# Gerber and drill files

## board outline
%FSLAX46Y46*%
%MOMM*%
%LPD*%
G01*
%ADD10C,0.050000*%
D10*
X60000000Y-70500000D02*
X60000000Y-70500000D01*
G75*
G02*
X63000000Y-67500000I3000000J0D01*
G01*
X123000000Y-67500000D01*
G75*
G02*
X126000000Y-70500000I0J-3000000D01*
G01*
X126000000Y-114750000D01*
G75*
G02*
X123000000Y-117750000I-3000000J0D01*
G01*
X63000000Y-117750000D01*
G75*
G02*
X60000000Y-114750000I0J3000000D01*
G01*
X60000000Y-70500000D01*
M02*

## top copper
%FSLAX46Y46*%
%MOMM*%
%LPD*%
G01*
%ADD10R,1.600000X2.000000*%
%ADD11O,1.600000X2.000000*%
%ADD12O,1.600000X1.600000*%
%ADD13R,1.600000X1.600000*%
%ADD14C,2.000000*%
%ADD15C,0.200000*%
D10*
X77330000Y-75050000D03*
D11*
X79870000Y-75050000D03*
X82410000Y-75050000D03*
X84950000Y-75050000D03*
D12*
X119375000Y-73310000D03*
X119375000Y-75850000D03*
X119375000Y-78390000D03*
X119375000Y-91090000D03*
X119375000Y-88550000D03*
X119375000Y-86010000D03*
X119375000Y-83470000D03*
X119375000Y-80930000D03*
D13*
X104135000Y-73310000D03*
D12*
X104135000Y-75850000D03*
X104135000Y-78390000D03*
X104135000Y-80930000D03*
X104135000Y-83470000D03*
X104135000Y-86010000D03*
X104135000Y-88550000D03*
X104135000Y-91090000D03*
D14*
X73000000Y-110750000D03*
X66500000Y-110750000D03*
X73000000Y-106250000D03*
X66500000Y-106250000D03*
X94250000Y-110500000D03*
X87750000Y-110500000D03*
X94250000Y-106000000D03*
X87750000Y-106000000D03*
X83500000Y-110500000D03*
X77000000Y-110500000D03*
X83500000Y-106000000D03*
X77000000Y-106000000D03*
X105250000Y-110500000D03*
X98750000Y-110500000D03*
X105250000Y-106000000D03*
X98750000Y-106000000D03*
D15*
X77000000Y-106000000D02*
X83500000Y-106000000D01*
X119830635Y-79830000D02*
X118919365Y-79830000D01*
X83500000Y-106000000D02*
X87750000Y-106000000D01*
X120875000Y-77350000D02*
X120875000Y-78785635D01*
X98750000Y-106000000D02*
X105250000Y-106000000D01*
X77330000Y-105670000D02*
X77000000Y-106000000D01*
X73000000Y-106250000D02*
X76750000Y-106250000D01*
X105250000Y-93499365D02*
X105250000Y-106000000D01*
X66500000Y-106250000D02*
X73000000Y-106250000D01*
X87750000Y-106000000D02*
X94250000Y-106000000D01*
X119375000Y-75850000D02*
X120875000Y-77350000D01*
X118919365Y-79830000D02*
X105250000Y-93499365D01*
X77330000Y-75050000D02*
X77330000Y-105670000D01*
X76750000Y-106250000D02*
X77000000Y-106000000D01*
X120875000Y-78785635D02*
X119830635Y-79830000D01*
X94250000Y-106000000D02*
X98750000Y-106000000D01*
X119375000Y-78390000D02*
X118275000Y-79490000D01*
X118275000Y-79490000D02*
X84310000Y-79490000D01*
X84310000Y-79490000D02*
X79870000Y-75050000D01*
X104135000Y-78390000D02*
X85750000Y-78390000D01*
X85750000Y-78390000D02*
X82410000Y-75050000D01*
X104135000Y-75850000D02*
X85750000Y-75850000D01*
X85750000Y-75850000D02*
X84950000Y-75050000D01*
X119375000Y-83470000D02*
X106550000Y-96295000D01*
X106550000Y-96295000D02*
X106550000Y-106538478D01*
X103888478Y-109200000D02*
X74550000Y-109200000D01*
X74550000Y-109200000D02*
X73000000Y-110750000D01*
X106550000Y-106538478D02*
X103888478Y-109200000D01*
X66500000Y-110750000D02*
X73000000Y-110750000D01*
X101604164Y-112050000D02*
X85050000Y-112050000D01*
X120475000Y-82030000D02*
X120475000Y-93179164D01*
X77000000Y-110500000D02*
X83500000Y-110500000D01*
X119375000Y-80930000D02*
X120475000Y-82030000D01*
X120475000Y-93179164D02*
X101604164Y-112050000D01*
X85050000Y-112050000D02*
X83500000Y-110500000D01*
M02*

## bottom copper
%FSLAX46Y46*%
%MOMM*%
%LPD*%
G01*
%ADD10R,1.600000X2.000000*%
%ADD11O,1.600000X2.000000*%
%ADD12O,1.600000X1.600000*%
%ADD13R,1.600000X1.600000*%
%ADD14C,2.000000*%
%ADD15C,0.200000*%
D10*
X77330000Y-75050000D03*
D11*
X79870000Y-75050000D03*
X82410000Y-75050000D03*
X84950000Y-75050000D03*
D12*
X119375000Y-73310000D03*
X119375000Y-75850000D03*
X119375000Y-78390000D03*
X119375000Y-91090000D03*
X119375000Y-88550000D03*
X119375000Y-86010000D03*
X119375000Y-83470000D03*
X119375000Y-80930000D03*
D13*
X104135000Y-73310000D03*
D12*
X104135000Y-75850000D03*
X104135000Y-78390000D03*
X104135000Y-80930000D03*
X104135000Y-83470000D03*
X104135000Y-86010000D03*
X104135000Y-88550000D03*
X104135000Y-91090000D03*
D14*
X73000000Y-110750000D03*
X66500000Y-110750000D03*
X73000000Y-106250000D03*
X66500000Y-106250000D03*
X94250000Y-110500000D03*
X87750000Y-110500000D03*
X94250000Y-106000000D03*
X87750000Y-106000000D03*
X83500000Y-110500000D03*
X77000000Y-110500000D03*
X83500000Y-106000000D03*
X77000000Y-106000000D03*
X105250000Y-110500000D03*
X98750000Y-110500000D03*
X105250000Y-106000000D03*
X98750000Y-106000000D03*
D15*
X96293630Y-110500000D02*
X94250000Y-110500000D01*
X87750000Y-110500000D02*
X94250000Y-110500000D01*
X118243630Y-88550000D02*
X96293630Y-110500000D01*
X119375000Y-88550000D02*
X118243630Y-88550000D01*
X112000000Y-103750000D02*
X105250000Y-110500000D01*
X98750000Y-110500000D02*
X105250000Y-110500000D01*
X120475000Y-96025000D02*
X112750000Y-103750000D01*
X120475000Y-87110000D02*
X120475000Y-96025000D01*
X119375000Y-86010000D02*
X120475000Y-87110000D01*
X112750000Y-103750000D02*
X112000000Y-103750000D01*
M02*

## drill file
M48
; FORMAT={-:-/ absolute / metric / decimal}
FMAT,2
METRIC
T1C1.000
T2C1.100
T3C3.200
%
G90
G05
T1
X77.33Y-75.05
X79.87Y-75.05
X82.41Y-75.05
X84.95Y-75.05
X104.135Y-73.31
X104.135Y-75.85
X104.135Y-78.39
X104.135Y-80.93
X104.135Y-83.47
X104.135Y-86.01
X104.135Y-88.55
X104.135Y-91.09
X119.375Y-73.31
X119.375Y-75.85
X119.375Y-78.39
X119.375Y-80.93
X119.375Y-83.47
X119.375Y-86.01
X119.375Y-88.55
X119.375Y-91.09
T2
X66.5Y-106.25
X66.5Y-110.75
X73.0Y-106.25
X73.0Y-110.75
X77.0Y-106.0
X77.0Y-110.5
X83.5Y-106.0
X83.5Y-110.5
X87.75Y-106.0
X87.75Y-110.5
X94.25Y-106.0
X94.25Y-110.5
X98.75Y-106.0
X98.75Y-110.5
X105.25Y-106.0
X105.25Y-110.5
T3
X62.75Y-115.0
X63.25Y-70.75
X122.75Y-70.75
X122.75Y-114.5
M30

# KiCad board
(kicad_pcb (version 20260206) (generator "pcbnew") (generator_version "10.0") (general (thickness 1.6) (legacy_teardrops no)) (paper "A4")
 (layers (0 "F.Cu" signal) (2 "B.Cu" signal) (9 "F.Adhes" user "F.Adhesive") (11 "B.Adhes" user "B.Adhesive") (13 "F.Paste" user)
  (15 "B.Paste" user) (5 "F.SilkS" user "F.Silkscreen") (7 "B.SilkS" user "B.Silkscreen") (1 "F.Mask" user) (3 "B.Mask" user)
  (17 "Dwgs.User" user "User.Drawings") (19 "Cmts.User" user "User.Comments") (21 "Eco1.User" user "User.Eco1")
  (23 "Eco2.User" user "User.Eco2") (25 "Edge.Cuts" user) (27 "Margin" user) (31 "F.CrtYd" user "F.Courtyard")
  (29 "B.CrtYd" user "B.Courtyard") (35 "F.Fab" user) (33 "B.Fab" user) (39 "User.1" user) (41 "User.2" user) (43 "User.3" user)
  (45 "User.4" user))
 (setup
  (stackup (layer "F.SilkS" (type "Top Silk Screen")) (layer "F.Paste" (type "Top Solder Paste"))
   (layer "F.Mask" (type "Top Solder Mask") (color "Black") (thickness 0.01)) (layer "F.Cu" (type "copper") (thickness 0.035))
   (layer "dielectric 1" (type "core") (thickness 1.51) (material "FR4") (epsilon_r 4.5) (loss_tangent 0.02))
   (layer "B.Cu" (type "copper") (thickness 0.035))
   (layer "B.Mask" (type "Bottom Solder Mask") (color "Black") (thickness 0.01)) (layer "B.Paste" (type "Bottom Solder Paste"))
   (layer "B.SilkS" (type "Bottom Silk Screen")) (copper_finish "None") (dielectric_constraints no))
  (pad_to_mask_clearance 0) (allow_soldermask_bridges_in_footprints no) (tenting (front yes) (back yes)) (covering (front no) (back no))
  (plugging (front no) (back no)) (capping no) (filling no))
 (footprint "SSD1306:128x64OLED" (layer "F.Cu") (at 80.95 85.65)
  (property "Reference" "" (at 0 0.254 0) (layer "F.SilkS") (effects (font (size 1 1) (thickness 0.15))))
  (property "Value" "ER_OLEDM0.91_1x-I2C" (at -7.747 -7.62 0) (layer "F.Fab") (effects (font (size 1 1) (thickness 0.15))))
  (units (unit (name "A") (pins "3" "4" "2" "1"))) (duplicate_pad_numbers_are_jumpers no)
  (pad "1" thru_hole rect (at -3.62 -10.6 90) (size 2 1.6) (drill 1) (layers "*.Cu" "*.Mask") (remove_unused_layers no) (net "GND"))
  (pad "2" thru_hole oval (at -1.08 -10.6 90) (size 2 1.6) (drill 1) (layers "*.Cu" "*.Mask") (remove_unused_layers no)
   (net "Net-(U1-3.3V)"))
  (pad "3" thru_hole oval (at 1.46 -10.6 90) (size 2 1.6) (drill 1) (layers "*.Cu" "*.Mask") (remove_unused_layers no) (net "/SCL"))
  (pad "4" thru_hole oval (at 4 -10.6 90) (size 2 1.6) (drill 1) (layers "*.Cu" "*.Mask") (remove_unused_layers no) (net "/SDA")))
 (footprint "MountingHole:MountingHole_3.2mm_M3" (layer "F.Cu") (at 122.75 114.5)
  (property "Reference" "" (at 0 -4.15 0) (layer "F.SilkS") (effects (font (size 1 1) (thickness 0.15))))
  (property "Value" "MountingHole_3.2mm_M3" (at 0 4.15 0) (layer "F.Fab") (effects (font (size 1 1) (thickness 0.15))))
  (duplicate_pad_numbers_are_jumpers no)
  (pad "" np_thru_hole circle (at 0 0) (size 3.2 3.2) (drill 3.2) (layers "*.Cu" "*.Mask")))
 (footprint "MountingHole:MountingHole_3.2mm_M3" (layer "F.Cu") (at 63.25 70.75)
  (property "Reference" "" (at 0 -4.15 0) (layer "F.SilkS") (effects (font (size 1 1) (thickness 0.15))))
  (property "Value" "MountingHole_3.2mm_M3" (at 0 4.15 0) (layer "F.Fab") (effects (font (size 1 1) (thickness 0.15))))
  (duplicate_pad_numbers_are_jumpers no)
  (pad "" np_thru_hole circle (at 0 0) (size 3.2 3.2) (drill 3.2) (layers "*.Cu" "*.Mask")))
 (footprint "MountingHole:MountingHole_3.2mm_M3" (layer "F.Cu") (at 62.75 115)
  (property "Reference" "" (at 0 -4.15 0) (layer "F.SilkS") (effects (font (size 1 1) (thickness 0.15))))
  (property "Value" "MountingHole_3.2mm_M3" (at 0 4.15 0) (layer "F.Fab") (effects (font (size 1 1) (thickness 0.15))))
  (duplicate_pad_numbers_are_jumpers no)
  (pad "" np_thru_hole circle (at 0 0) (size 3.2 3.2) (drill 3.2) (layers "*.Cu" "*.Mask")))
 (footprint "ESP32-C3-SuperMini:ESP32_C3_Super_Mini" (layer "F.Cu") (at 104.135 73.31)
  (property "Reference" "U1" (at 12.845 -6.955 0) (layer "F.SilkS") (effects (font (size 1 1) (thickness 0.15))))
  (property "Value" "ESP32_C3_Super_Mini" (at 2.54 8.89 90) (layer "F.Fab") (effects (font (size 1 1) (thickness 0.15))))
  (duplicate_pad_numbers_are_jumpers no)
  (pad "-1" thru_hole oval (at 15.24 0) (size 1.6 1.6) (drill 1) (layers "*.Cu" "*.Mask") (remove_unused_layers no) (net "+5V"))
  (pad "-2" thru_hole oval (at 15.24 2.54) (size 1.6 1.6) (drill 1) (layers "*.Cu" "*.Mask") (remove_unused_layers no) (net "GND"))
  (pad "-3" thru_hole oval (at 15.24 5.08) (size 1.6 1.6) (drill 1) (layers "*.Cu" "*.Mask") (remove_unused_layers no) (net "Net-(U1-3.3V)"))
  (pad "0" thru_hole oval (at 15.24 17.78) (size 1.6 1.6) (drill 1) (layers "*.Cu" "*.Mask") (remove_unused_layers no)
   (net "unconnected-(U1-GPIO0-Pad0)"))
  (pad "1" thru_hole oval (at 15.24 15.24) (size 1.6 1.6) (drill 1) (layers "*.Cu" "*.Mask") (remove_unused_layers no) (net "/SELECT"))
  (pad "2" thru_hole oval (at 15.24 12.7) (size 1.6 1.6) (drill 1) (layers "*.Cu" "*.Mask") (remove_unused_layers no) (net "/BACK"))
  (pad "3" thru_hole oval (at 15.24 10.16) (size 1.6 1.6) (drill 1) (layers "*.Cu" "*.Mask") (remove_unused_layers no) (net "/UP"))
  (pad "4" thru_hole oval (at 15.24 7.62) (size 1.6 1.6) (drill 1) (layers "*.Cu" "*.Mask") (remove_unused_layers no) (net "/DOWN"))
  (pad "5" thru_hole rect (at 0 0) (size 1.6 1.6) (drill 1) (layers "*.Cu" "*.Mask") (remove_unused_layers no)
   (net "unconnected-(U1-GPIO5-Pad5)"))
  (pad "6" thru_hole oval (at 0 2.54) (size 1.6 1.6) (drill 1) (layers "*.Cu" "*.Mask") (remove_unused_layers no) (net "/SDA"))
  (pad "7" thru_hole oval (at 0 5.08) (size 1.6 1.6) (drill 1) (layers "*.Cu" "*.Mask") (remove_unused_layers no) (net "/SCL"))
  (pad "8" thru_hole oval (at 0 7.62) (size 1.6 1.6) (drill 1) (layers "*.Cu" "*.Mask") (remove_unused_layers no)
   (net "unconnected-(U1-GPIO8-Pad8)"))
  (pad "9" thru_hole oval (at 0 10.16) (size 1.6 1.6) (drill 1) (layers "*.Cu" "*.Mask") (remove_unused_layers no)
   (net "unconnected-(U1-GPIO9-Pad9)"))
  (pad "10" thru_hole oval (at 0 12.7) (size 1.6 1.6) (drill 1) (layers "*.Cu" "*.Mask") (remove_unused_layers no)
   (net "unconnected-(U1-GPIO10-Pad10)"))
  (pad "20" thru_hole oval (at 0 15.24) (size 1.6 1.6) (drill 1) (layers "*.Cu" "*.Mask") (remove_unused_layers no)
   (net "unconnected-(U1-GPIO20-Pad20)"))
  (pad "21" thru_hole oval (at 0 17.78) (size 1.6 1.6) (drill 1) (layers "*.Cu" "*.Mask") (remove_unused_layers no)
   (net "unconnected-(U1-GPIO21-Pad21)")))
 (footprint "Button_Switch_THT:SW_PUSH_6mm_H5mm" (layer "F.Cu") (at 73 110.75 180)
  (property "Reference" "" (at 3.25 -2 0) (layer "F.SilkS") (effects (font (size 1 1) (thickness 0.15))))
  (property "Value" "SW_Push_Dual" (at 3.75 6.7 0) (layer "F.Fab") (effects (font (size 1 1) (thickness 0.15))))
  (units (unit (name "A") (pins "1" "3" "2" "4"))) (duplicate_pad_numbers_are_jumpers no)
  (pad "1" thru_hole circle (at 0 0 270) (size 2 2) (drill 1.1) (layers "*.Cu" "*.Mask") (remove_unused_layers no) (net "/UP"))
  (pad "1" thru_hole circle (at 6.5 0 270) (size 2 2) (drill 1.1) (layers "*.Cu" "*.Mask") (remove_unused_layers no) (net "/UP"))
  (pad "2" thru_hole circle (at 0 4.5 270) (size 2 2) (drill 1.1) (layers "*.Cu" "*.Mask") (remove_unused_layers no) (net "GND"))
  (pad "2" thru_hole circle (at 6.5 4.5 270) (size 2 2) (drill 1.1) (layers "*.Cu" "*.Mask") (remove_unused_layers no) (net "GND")))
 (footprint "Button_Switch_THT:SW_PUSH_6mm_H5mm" (layer "F.Cu") (at 94.25 110.5 180)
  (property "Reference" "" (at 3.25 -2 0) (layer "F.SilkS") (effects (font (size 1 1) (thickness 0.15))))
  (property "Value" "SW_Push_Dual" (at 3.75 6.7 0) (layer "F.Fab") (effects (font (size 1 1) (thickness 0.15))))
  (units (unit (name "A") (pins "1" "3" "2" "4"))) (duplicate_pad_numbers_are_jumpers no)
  (pad "1" thru_hole circle (at 0 0 270) (size 2 2) (drill 1.1) (layers "*.Cu" "*.Mask") (remove_unused_layers no) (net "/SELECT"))
  (pad "1" thru_hole circle (at 6.5 0 270) (size 2 2) (drill 1.1) (layers "*.Cu" "*.Mask") (remove_unused_layers no) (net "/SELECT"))
  (pad "2" thru_hole circle (at 0 4.5 270) (size 2 2) (drill 1.1) (layers "*.Cu" "*.Mask") (remove_unused_layers no) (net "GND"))
  (pad "2" thru_hole circle (at 6.5 4.5 270) (size 2 2) (drill 1.1) (layers "*.Cu" "*.Mask") (remove_unused_layers no) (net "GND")))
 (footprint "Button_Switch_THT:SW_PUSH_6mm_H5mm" (layer "F.Cu") (at 83.5 110.5 180)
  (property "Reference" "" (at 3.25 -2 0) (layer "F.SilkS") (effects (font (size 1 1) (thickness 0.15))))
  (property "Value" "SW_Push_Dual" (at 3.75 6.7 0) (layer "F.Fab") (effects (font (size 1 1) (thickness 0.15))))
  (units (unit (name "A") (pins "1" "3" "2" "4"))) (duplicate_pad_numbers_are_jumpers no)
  (pad "1" thru_hole circle (at 0 0 270) (size 2 2) (drill 1.1) (layers "*.Cu" "*.Mask") (remove_unused_layers no) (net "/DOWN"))
  (pad "1" thru_hole circle (at 6.5 0 270) (size 2 2) (drill 1.1) (layers "*.Cu" "*.Mask") (remove_unused_layers no) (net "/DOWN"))
  (pad "2" thru_hole circle (at 0 4.5 270) (size 2 2) (drill 1.1) (layers "*.Cu" "*.Mask") (remove_unused_layers no) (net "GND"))
  (pad "2" thru_hole circle (at 6.5 4.5 270) (size 2 2) (drill 1.1) (layers "*.Cu" "*.Mask") (remove_unused_layers no) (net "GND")))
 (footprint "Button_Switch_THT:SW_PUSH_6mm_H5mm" (layer "F.Cu") (at 105.25 110.5 180)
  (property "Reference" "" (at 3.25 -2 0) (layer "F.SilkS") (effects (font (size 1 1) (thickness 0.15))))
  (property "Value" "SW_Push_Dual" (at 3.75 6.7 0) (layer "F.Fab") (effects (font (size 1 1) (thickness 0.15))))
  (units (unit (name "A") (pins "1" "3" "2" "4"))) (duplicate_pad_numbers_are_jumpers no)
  (pad "1" thru_hole circle (at 0 0 270) (size 2 2) (drill 1.1) (layers "*.Cu" "*.Mask") (remove_unused_layers no) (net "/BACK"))
  (pad "1" thru_hole circle (at 6.5 0 270) (size 2 2) (drill 1.1) (layers "*.Cu" "*.Mask") (remove_unused_layers no) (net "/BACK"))
  (pad "2" thru_hole circle (at 0 4.5 270) (size 2 2) (drill 1.1) (layers "*.Cu" "*.Mask") (remove_unused_layers no) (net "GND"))
  (pad "2" thru_hole circle (at 6.5 4.5 270) (size 2 2) (drill 1.1) (layers "*.Cu" "*.Mask") (remove_unused_layers no) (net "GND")))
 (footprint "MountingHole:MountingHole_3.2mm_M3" (layer "F.Cu") (at 122.75 70.75)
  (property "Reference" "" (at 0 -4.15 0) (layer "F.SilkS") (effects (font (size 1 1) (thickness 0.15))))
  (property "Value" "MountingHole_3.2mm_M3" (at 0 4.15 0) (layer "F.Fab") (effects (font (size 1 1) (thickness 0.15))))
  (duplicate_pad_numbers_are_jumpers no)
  (pad "" np_thru_hole circle (at 0 0) (size 3.2 3.2) (drill 3.2) (layers "*.Cu" "*.Mask")))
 (gr_rect (start 60 67.5) (end 126 117.75) (radius 3) (stroke (width 0.05) (type default)) (fill no) (layer "Edge.Cuts"))
 (segment (start 77 106) (end 83.5 106) (width 0.2) (layer "F.Cu") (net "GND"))
 (segment (start 119.830635 79.83) (end 118.919365 79.83) (width 0.2) (layer "F.Cu") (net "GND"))
 (segment (start 83.5 106) (end 87.75 106) (width 0.2) (layer "F.Cu") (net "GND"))
 (segment (start 120.875 77.35) (end 120.875 78.785635) (width 0.2) (layer "F.Cu") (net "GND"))
 (segment (start 98.75 106) (end 105.25 106) (width 0.2) (layer "F.Cu") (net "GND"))
 (segment (start 77.33 105.67) (end 77 106) (width 0.2) (layer "F.Cu") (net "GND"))
 (segment (start 73 106.25) (end 76.75 106.25) (width 0.2) (layer "F.Cu") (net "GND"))
 (segment (start 105.25 93.499365) (end 105.25 106) (width 0.2) (layer "F.Cu") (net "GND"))
 (segment (start 66.5 106.25) (end 73 106.25) (width 0.2) (layer "F.Cu") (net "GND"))
 (segment (start 87.75 106) (end 94.25 106) (width 0.2) (layer "F.Cu") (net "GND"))
 (segment (start 119.375 75.85) (end 120.875 77.35) (width 0.2) (layer "F.Cu") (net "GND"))
 (segment (start 118.919365 79.83) (end 105.25 93.499365) (width 0.2) (layer "F.Cu") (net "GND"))
 (segment (start 77.33 75.05) (end 77.33 105.67) (width 0.2) (layer "F.Cu") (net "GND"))
 (segment (start 76.75 106.25) (end 77 106) (width 0.2) (layer "F.Cu") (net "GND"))
 (segment (start 120.875 78.785635) (end 119.830635 79.83) (width 0.2) (layer "F.Cu") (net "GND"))
 (segment (start 94.25 106) (end 98.75 106) (width 0.2) (layer "F.Cu") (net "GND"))
 (segment (start 119.375 78.39) (end 118.275 79.49) (width 0.2) (layer "F.Cu") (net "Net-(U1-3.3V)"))
 (segment (start 118.275 79.49) (end 84.31 79.49) (width 0.2) (layer "F.Cu") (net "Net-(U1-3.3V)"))
 (segment (start 84.31 79.49) (end 79.87 75.05) (width 0.2) (layer "F.Cu") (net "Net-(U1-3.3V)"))
 (segment (start 104.135 78.39) (end 85.75 78.39) (width 0.2) (layer "F.Cu") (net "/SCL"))
 (segment (start 85.75 78.39) (end 82.41 75.05) (width 0.2) (layer "F.Cu") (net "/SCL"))
 (segment (start 104.135 75.85) (end 85.75 75.85) (width 0.2) (layer "F.Cu") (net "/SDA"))
 (segment (start 85.75 75.85) (end 84.95 75.05) (width 0.2) (layer "F.Cu") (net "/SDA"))
 (segment (start 96.29363 110.5) (end 94.25 110.5) (width 0.2) (layer "B.Cu") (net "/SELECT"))
 (segment (start 87.75 110.5) (end 94.25 110.5) (width 0.2) (layer "B.Cu") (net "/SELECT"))
 (segment (start 118.24363 88.55) (end 96.29363 110.5) (width 0.2) (layer "B.Cu") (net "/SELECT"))
 (segment (start 119.375 88.55) (end 118.24363 88.55) (width 0.2) (layer "B.Cu") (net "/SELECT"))
 (segment (start 112 103.75) (end 105.25 110.5) (width 0.2) (layer "B.Cu") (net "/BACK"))
 (segment (start 98.75 110.5) (end 105.25 110.5) (width 0.2) (layer "B.Cu") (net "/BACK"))
 (segment (start 120.475 96.025) (end 112.75 103.75) (width 0.2) (layer "B.Cu") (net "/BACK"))
 (segment (start 120.475 87.11) (end 120.475 96.025) (width 0.2) (layer "B.Cu") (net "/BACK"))
 (segment (start 119.375 86.01) (end 120.475 87.11) (width 0.2) (layer "B.Cu") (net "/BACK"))
 (segment (start 112.75 103.75) (end 112 103.75) (width 0.2) (layer "B.Cu") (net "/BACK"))
 (segment (start 119.375 83.47) (end 106.55 96.295) (width 0.2) (layer "F.Cu") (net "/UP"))
 (segment (start 106.55 96.295) (end 106.55 106.538478) (width 0.2) (layer "F.Cu") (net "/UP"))
 (segment (start 103.888478 109.2) (end 74.55 109.2) (width 0.2) (layer "F.Cu") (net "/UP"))
 (segment (start 74.55 109.2) (end 73 110.75) (width 0.2) (layer "F.Cu") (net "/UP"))
 (segment (start 106.55 106.538478) (end 103.888478 109.2) (width 0.2) (layer "F.Cu") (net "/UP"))
 (segment (start 66.5 110.75) (end 73 110.75) (width 0.2) (layer "F.Cu") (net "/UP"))
 (segment (start 101.604164 112.05) (end 85.05 112.05) (width 0.2) (layer "F.Cu") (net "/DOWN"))
 (segment (start 120.475 82.03) (end 120.475 93.179164) (width 0.2) (layer "F.Cu") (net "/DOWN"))
 (segment (start 77 110.5) (end 83.5 110.5) (width 0.2) (layer "F.Cu") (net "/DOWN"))
 (segment (start 119.375 80.93) (end 120.475 82.03) (width 0.2) (layer "F.Cu") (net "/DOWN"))
 (segment (start 120.475 93.179164) (end 101.604164 112.05) (width 0.2) (layer "F.Cu") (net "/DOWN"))
 (segment (start 85.05 112.05) (end 83.5 110.5) (width 0.2) (layer "F.Cu") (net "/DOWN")))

